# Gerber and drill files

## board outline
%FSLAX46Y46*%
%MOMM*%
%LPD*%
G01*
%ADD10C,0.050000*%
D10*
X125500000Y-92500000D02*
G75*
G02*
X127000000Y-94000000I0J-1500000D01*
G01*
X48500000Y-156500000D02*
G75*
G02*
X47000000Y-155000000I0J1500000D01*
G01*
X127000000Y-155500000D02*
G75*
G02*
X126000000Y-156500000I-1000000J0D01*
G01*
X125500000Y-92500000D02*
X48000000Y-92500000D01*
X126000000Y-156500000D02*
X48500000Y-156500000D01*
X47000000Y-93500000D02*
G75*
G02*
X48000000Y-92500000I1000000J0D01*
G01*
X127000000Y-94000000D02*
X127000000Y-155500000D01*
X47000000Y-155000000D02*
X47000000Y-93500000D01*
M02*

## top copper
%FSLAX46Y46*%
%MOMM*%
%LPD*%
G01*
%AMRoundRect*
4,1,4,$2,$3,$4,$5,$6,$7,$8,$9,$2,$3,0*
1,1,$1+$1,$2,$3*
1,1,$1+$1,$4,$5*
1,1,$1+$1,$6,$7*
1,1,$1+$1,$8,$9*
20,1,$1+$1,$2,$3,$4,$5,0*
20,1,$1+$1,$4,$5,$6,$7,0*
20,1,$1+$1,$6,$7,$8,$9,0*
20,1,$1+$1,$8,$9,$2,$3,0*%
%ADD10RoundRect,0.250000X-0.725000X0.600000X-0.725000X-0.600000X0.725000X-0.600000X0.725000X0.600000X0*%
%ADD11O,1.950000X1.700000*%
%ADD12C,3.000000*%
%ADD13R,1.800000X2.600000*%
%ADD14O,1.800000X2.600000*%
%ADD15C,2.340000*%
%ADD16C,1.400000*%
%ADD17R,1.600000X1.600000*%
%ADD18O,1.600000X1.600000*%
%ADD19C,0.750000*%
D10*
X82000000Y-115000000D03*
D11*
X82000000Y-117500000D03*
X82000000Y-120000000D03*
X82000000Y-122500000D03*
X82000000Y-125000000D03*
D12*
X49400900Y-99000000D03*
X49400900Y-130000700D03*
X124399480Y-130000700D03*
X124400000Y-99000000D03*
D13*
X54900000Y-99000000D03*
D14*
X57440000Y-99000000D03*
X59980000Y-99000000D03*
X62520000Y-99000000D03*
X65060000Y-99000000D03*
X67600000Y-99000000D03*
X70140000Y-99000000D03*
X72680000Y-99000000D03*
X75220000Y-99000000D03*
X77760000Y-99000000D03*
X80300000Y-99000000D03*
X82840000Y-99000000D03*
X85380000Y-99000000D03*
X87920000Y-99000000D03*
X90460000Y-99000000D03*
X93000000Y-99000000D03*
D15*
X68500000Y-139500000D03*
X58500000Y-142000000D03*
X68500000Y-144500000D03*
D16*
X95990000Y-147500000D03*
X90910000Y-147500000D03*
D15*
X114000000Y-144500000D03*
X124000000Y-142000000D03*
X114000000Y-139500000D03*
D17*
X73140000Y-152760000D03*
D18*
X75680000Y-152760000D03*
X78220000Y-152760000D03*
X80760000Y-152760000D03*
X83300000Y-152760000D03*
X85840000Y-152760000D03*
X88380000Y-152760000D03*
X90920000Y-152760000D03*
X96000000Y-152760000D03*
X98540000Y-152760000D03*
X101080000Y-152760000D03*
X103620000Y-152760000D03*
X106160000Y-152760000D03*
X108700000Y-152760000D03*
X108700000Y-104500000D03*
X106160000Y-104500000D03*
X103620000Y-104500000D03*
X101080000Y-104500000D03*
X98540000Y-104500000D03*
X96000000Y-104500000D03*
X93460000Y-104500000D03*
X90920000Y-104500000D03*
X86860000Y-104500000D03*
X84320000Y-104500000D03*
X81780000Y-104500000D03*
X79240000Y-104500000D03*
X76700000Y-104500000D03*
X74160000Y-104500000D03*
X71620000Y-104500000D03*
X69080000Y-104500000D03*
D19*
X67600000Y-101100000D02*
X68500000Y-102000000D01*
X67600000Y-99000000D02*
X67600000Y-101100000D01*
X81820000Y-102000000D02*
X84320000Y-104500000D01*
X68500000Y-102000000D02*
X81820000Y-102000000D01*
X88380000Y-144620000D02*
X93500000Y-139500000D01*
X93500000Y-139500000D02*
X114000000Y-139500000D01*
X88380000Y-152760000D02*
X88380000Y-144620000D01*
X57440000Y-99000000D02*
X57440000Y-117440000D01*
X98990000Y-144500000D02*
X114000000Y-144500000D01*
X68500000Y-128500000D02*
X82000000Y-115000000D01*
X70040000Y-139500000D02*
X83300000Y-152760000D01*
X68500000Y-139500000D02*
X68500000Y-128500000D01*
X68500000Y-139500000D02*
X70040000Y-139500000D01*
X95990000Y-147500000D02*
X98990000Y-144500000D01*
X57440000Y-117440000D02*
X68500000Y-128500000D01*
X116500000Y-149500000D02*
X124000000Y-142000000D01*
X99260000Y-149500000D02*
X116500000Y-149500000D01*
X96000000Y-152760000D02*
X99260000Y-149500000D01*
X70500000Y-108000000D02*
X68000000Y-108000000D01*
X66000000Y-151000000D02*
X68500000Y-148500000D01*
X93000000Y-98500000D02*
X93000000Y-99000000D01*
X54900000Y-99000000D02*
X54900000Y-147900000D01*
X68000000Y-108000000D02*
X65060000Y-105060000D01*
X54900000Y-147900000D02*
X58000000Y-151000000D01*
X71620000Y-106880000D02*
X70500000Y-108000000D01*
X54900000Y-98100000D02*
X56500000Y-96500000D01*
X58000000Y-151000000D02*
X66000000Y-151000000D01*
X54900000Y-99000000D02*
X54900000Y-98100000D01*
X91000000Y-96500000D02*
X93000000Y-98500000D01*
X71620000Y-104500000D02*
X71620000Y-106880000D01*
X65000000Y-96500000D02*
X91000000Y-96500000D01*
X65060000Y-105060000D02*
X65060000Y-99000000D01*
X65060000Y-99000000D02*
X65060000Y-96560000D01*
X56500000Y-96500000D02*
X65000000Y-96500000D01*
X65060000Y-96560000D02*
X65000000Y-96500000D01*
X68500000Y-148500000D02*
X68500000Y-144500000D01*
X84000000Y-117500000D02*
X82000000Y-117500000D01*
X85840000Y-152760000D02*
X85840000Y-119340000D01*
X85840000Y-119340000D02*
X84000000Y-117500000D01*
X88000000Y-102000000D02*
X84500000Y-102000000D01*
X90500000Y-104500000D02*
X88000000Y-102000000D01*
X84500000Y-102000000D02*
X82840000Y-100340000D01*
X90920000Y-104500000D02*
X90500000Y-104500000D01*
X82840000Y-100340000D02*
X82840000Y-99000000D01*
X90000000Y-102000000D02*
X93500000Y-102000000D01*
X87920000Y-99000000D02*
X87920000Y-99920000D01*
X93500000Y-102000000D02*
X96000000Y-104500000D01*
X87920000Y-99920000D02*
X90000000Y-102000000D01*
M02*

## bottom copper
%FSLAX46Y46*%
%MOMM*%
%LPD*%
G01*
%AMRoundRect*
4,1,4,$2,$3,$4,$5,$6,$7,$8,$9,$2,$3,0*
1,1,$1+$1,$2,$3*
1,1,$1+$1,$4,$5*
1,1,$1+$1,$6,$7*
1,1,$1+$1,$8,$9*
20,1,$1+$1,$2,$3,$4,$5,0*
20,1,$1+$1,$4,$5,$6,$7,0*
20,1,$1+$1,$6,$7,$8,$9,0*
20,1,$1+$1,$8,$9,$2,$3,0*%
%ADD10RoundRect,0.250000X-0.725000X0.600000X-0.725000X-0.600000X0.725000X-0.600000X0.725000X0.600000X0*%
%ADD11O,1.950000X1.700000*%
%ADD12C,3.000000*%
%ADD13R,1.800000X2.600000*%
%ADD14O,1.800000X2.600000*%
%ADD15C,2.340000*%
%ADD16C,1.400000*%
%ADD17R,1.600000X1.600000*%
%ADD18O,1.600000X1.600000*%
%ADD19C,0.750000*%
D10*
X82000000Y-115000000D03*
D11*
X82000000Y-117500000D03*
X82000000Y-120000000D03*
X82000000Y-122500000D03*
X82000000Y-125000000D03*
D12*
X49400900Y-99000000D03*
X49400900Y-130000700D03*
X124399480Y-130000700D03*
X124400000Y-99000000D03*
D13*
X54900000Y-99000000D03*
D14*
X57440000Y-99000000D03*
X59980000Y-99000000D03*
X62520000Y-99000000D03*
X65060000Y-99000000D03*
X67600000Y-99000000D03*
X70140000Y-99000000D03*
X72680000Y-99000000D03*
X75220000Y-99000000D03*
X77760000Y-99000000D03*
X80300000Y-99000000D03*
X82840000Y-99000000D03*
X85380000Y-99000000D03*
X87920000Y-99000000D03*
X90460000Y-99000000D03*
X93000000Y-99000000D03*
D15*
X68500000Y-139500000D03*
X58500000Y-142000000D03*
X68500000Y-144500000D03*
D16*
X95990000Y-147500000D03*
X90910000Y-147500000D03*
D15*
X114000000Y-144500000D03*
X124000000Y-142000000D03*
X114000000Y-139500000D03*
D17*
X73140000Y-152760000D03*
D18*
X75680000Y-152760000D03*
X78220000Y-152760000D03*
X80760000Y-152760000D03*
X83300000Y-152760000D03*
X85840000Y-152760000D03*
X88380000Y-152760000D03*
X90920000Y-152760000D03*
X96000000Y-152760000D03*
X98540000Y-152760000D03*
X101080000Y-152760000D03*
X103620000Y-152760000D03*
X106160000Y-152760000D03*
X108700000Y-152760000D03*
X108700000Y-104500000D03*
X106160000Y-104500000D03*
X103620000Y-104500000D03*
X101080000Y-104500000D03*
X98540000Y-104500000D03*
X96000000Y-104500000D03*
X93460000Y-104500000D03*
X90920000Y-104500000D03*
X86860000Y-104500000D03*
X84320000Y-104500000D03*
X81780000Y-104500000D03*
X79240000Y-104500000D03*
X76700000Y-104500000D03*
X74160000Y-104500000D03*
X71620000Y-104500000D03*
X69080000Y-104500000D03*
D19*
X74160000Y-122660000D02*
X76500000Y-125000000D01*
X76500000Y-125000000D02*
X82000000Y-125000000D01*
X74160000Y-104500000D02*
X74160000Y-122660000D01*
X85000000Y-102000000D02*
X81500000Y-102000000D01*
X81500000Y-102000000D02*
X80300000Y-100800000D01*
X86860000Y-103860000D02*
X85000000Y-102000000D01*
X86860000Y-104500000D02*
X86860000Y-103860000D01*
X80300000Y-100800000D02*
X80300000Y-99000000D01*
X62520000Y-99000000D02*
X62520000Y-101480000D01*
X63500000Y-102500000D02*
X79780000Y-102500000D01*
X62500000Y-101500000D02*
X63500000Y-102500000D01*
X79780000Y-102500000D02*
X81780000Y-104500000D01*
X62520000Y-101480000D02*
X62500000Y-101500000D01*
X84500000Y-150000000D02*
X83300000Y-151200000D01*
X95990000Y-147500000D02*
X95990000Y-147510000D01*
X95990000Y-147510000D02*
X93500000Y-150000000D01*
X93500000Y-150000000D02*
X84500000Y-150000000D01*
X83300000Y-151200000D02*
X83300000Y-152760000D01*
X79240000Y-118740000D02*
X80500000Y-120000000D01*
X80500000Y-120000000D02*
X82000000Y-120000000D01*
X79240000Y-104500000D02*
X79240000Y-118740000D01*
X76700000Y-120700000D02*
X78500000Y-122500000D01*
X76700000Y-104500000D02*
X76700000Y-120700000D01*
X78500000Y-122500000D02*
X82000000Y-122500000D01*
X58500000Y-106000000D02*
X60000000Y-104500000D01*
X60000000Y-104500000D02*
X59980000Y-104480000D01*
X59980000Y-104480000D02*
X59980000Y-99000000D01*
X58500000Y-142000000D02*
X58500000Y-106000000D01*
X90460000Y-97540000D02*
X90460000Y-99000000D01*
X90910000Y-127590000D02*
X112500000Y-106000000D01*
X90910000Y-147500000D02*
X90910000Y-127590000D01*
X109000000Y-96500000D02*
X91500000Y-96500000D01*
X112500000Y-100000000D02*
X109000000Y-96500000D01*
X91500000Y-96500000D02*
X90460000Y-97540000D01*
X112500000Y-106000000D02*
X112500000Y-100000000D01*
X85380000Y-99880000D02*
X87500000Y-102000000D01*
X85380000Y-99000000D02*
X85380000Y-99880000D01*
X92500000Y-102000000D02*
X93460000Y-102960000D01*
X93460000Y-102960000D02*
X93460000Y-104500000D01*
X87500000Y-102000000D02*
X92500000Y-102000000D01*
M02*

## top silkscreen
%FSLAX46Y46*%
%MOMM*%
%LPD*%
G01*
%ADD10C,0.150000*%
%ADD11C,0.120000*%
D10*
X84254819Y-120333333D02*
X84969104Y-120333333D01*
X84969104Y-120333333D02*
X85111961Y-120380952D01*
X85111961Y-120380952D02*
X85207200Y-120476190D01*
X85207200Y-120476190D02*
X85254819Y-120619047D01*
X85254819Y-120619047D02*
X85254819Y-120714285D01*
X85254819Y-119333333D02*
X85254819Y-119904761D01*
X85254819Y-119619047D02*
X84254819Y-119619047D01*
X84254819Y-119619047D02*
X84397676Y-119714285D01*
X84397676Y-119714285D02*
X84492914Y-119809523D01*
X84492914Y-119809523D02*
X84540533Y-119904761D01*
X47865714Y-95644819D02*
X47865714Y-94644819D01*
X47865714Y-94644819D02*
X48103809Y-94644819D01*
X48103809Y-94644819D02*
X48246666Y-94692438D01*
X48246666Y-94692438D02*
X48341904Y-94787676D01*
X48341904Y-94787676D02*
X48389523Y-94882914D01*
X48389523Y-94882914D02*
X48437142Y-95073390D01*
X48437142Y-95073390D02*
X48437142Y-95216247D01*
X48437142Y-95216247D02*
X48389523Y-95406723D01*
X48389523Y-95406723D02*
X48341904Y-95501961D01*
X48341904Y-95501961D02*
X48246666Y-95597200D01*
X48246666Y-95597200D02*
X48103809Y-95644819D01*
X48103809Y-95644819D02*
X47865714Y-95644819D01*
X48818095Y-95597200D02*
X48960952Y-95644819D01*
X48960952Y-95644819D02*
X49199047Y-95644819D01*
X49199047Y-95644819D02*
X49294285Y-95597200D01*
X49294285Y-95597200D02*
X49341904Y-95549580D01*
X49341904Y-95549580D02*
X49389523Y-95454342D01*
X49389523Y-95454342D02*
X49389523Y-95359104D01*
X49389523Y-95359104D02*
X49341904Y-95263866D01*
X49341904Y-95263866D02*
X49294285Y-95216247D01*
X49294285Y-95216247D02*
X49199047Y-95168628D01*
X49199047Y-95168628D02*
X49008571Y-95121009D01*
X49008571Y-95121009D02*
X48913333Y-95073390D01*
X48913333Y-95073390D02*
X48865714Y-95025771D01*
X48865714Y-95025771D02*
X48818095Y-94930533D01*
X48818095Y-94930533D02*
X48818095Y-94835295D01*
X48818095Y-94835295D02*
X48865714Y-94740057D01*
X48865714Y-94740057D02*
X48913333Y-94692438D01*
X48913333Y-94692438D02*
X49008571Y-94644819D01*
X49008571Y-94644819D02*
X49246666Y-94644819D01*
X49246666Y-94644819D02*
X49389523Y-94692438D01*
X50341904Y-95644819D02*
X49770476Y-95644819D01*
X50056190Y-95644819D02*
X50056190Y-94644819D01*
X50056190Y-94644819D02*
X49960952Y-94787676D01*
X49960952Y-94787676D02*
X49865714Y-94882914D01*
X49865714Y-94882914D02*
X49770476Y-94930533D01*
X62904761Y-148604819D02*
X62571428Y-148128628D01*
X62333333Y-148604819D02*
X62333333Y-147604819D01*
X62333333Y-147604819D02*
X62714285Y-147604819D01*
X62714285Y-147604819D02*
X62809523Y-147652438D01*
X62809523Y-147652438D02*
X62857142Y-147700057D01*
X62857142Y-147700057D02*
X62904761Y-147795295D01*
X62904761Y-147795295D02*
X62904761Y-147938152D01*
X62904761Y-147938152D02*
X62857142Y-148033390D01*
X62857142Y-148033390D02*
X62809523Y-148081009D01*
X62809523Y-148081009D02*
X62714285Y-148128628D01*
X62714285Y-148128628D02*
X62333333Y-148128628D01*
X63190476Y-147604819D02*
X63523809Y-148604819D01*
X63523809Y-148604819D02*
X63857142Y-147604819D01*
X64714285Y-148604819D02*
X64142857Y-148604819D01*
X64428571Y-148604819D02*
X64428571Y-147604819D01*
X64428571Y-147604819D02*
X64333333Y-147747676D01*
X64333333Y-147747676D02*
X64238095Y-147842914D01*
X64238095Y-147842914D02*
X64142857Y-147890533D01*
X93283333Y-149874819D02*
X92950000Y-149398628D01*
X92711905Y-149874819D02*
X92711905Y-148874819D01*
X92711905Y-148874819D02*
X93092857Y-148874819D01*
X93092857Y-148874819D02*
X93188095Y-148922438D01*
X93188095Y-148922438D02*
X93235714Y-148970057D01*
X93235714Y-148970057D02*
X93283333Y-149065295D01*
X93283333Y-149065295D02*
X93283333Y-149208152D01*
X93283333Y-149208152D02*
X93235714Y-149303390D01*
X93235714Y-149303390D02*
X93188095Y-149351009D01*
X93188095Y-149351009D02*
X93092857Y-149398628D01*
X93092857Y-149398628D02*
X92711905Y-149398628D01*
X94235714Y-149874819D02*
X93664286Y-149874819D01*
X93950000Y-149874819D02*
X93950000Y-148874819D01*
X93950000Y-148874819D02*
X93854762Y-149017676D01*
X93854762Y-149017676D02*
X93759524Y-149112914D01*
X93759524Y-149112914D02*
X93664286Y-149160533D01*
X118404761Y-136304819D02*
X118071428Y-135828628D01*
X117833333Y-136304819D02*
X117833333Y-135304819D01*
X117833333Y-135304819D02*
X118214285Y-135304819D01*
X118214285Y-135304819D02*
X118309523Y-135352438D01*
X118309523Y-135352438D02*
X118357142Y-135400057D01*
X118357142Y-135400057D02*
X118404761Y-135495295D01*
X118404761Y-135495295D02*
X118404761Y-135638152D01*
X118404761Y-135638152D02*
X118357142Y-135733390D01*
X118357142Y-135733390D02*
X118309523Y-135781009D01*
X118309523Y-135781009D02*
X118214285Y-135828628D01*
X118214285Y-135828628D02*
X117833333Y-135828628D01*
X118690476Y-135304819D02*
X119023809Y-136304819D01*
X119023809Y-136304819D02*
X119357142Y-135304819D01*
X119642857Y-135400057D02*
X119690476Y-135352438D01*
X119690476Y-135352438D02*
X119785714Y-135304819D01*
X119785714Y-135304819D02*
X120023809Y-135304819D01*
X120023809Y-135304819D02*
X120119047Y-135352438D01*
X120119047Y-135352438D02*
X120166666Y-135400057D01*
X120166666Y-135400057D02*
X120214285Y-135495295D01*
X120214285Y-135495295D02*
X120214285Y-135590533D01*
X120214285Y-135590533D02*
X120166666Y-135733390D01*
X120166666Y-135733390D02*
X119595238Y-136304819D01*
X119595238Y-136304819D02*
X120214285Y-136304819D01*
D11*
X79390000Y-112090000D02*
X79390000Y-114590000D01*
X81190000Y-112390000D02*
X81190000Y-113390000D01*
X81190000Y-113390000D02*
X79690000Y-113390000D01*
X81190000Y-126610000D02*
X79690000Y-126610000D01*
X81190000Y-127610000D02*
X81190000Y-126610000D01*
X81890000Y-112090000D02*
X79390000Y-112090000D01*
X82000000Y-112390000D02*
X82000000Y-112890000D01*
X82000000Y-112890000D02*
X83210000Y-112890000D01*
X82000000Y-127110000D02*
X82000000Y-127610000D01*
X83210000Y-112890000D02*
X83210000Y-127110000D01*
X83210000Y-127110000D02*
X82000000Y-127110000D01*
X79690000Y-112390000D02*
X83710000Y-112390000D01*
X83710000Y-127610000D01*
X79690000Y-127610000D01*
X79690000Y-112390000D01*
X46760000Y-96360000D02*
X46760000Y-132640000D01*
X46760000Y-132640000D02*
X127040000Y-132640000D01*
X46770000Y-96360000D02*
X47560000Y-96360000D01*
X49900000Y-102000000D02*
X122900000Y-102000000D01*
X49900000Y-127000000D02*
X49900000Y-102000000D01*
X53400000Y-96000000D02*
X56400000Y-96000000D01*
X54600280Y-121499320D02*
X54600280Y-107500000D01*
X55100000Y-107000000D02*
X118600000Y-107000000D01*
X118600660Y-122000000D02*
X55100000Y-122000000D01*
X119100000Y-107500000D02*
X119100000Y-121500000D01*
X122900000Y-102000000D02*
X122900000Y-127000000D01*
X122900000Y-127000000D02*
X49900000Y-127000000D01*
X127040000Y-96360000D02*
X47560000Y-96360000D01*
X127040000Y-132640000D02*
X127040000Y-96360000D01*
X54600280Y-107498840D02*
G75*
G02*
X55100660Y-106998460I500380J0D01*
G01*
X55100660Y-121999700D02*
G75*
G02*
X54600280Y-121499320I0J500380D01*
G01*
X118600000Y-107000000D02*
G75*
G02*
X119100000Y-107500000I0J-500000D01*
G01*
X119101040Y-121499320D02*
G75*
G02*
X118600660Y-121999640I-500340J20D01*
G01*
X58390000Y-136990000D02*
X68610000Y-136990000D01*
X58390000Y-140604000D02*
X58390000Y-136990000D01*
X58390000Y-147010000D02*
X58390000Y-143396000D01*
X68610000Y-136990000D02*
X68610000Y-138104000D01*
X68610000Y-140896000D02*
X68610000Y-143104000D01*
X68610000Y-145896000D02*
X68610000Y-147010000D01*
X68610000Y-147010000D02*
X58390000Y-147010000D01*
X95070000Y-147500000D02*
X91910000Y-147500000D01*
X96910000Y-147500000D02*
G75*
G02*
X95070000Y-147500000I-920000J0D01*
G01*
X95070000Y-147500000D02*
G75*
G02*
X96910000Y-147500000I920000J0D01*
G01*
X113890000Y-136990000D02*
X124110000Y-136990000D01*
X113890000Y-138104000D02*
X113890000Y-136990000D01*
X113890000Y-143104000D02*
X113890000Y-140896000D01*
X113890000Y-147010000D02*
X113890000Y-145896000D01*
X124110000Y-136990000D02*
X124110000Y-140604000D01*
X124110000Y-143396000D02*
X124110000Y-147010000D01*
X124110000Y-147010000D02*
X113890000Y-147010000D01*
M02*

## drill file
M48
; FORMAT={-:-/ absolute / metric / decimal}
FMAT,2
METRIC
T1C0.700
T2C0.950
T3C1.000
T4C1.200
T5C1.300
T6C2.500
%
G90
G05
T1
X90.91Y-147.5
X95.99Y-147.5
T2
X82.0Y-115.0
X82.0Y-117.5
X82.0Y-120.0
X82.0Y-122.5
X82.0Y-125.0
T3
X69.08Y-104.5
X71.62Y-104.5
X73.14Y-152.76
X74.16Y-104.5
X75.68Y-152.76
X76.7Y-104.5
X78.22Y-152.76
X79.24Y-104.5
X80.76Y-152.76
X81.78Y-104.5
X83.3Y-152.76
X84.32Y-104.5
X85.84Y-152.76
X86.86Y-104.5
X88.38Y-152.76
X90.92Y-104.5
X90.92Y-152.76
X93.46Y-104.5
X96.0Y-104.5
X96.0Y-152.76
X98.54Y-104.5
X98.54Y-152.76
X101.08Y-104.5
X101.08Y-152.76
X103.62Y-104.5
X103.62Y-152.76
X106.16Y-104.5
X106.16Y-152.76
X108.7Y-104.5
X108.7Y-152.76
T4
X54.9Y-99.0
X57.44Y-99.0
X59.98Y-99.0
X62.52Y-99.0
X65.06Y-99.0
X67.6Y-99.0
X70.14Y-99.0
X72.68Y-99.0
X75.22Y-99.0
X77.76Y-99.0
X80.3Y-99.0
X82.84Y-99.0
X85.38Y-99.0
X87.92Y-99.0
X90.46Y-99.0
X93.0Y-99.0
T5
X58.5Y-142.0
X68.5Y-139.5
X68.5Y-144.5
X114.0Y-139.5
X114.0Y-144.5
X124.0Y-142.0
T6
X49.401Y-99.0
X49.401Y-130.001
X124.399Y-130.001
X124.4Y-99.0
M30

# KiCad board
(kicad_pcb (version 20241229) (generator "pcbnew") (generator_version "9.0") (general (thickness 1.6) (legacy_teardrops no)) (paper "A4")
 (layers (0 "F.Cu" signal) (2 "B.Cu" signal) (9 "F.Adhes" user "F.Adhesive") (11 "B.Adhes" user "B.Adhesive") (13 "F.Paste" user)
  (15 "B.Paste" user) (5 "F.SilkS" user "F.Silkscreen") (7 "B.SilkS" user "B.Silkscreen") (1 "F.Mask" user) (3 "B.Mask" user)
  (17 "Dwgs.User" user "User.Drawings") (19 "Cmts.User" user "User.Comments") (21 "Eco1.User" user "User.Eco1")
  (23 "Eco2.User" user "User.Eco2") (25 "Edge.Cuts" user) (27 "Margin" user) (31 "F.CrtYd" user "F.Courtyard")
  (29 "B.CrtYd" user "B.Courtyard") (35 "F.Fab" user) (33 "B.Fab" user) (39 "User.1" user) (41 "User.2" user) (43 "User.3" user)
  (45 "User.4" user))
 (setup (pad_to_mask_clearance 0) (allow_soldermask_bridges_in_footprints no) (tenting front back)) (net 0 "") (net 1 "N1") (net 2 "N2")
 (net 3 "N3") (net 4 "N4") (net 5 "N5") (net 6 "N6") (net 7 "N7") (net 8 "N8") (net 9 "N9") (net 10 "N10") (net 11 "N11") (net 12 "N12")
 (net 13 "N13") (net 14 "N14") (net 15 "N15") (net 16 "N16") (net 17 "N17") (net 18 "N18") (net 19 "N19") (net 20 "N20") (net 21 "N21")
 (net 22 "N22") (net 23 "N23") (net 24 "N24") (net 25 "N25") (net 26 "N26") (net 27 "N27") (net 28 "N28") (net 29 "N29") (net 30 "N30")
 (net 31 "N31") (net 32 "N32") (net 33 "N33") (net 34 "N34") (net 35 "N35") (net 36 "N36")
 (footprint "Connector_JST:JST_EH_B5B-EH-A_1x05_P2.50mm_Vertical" (layer "F.Cu") (at 82 115 -90)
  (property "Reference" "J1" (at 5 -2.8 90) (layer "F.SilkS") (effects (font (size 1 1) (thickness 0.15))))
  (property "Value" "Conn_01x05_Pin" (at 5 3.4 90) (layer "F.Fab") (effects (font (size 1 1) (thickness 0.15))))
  (fp_line (start -2.91 2.61) (end -0.41 2.61) (stroke (width 0.12) (type solid)) (layer "F.SilkS"))
  (fp_line (start -2.61 0.81) (end -1.61 0.81) (stroke (width 0.12) (type solid)) (layer "F.SilkS"))
  (fp_line (start -1.61 0.81) (end -1.61 2.31) (stroke (width 0.12) (type solid)) (layer "F.SilkS"))
  (fp_line (start 11.61 0.81) (end 11.61 2.31) (stroke (width 0.12) (type solid)) (layer "F.SilkS"))
  (fp_line (start 12.61 0.81) (end 11.61 0.81) (stroke (width 0.12) (type solid)) (layer "F.SilkS"))
  (fp_line (start -2.91 0.11) (end -2.91 2.61) (stroke (width 0.12) (type solid)) (layer "F.SilkS"))
  (fp_line (start -2.61 0) (end -2.11 0) (stroke (width 0.12) (type solid)) (layer "F.SilkS"))
  (fp_line (start -2.11 0) (end -2.11 -1.21) (stroke (width 0.12) (type solid)) (layer "F.SilkS"))
  (fp_line (start 12.11 0) (end 12.61 0) (stroke (width 0.12) (type solid)) (layer "F.SilkS"))
  (fp_line (start -2.11 -1.21) (end 12.11 -1.21) (stroke (width 0.12) (type solid)) (layer "F.SilkS"))
  (fp_line (start 12.11 -1.21) (end 12.11 0) (stroke (width 0.12) (type solid)) (layer "F.SilkS"))
  (fp_rect (start -2.61 -1.71) (end 12.61 2.31) (stroke (width 0.12) (type solid)) (fill no) (layer "F.SilkS"))
  (pad "1" thru_hole roundrect (at 0 0 270) (size 1.7 1.95) (drill 0.95) (layers "*.Cu" "*.Mask") (remove_unused_layers no)
   (roundrect_rratio 0.147059) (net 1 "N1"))
  (pad "2" thru_hole oval (at 2.5 0 270) (size 1.7 1.95) (drill 0.95) (layers "*.Cu" "*.Mask") (remove_unused_layers no) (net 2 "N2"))
  (pad "3" thru_hole oval (at 5 0 270) (size 1.7 1.95) (drill 0.95) (layers "*.Cu" "*.Mask") (remove_unused_layers no) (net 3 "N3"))
  (pad "4" thru_hole oval (at 7.5 0 270) (size 1.7 1.95) (drill 0.95) (layers "*.Cu" "*.Mask") (remove_unused_layers no) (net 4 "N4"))
  (pad "5" thru_hole oval (at 10 0 270) (size 1.7 1.95) (drill 0.95) (layers "*.Cu" "*.Mask") (remove_unused_layers no) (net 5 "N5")))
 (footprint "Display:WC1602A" (layer "F.Cu") (at 54.9 99)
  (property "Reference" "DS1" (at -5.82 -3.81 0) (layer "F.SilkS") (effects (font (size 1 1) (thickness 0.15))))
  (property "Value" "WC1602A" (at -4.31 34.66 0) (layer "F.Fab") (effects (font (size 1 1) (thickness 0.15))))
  (fp_line (start -8.14 -2.64) (end -8.14 33.64) (stroke (width 0.12) (type solid)) (layer "F.SilkS"))
  (fp_line (start -8.14 33.64) (end 72.14 33.64) (stroke (width 0.12) (type solid)) (layer "F.SilkS"))
  (fp_line (start -8.13 -2.64) (end -7.34 -2.64) (stroke (width 0.12) (type solid)) (layer "F.SilkS"))
  (fp_line (start -5 3) (end 68 3) (stroke (width 0.12) (type solid)) (layer "F.SilkS"))
  (fp_line (start -5 28) (end -5 3) (stroke (width 0.12) (type solid)) (layer "F.SilkS"))
  (fp_line (start -1.5 -3) (end 1.5 -3) (stroke (width 0.12) (type solid)) (layer "F.SilkS"))
  (fp_line (start -0.29972 22.49932) (end -0.29972 8.5) (stroke (width 0.12) (type solid)) (layer "F.SilkS"))
  (fp_line (start 0.2 8) (end 63.7 8) (stroke (width 0.12) (type solid)) (layer "F.SilkS"))
  (fp_line (start 63.70066 23) (end 0.2 23) (stroke (width 0.12) (type solid)) (layer "F.SilkS"))
  (fp_line (start 64.2 8.5) (end 64.2 22.5) (stroke (width 0.12) (type solid)) (layer "F.SilkS"))
  (fp_line (start 68 3) (end 68 28) (stroke (width 0.12) (type solid)) (layer "F.SilkS"))
  (fp_line (start 68 28) (end -5 28) (stroke (width 0.12) (type solid)) (layer "F.SilkS"))
  (fp_line (start 72.14 -2.64) (end -7.34 -2.64) (stroke (width 0.12) (type solid)) (layer "F.SilkS"))
  (fp_line (start 72.14 33.64) (end 72.14 -2.64) (stroke (width 0.12) (type solid)) (layer "F.SilkS"))
  (fp_arc (start -0.29972 8.49884) (mid -0.153162 8.145018) (end 0.20066 7.99846) (stroke (width 0.12) (type solid)) (layer "F.SilkS"))
  (fp_arc (start 0.20066 22.9997) (mid -0.153162 22.853142) (end -0.29972 22.49932) (stroke (width 0.12) (type solid)) (layer "F.SilkS"))
  (fp_arc (start 63.7 8) (mid 64.053553 8.146447) (end 64.2 8.5) (stroke (width 0.12) (type solid)) (layer "F.SilkS"))
  (fp_arc (start 64.20104 22.49932) (mid 64.054482 22.853142) (end 63.70066 22.9997) (stroke (width 0.12) (type solid)) (layer "F.SilkS"))
  (pad "" thru_hole circle (at -5.4991 0) (size 3 3) (drill 2.5) (layers "*.Cu" "*.Mask") (remove_unused_layers no))
  (pad "" thru_hole circle (at -5.4991 31.0007) (size 3 3) (drill 2.5) (layers "*.Cu" "*.Mask") (remove_unused_layers no))
  (pad "" thru_hole circle (at 69.49948 31.0007) (size 3 3) (drill 2.5) (layers "*.Cu" "*.Mask") (remove_unused_layers no))
  (pad "" thru_hole circle (at 69.5 0) (size 3 3) (drill 2.5) (layers "*.Cu" "*.Mask") (remove_unused_layers no))
  (pad "1" thru_hole rect (at 0 0) (size 1.8 2.6) (drill 1.2) (layers "*.Cu" "*.Mask") (remove_unused_layers no) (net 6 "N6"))
  (pad "2" thru_hole oval (at 2.54 0) (size 1.8 2.6) (drill 1.2) (layers "*.Cu" "*.Mask") (remove_unused_layers no) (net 1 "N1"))
  (pad "3" thru_hole oval (at 5.08 0) (size 1.8 2.6) (drill 1.2) (layers "*.Cu" "*.Mask") (remove_unused_layers no) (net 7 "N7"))
  (pad "4" thru_hole oval (at 7.62 0) (size 1.8 2.6) (drill 1.2) (layers "*.Cu" "*.Mask") (remove_unused_layers no) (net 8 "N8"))
  (pad "5" thru_hole oval (at 10.16 0) (size 1.8 2.6) (drill 1.2) (layers "*.Cu" "*.Mask") (remove_unused_layers no) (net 6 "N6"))
  (pad "6" thru_hole oval (at 12.7 0) (size 1.8 2.6) (drill 1.2) (layers "*.Cu" "*.Mask") (remove_unused_layers no) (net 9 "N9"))
  (pad "7" thru_hole oval (at 15.24 0) (size 1.8 2.6) (drill 1.2) (layers "*.Cu" "*.Mask") (remove_unused_layers no) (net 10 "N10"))
  (pad "8" thru_hole oval (at 17.78 0) (size 1.8 2.6) (drill 1.2) (layers "*.Cu" "*.Mask") (remove_unused_layers no) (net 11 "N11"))
  (pad "9" thru_hole oval (at 20.32 0) (size 1.8 2.6) (drill 1.2) (layers "*.Cu" "*.Mask") (remove_unused_layers no) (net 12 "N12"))
  (pad "10" thru_hole oval (at 22.86 0) (size 1.8 2.6) (drill 1.2) (layers "*.Cu" "*.Mask") (remove_unused_layers no) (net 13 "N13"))
  (pad "11" thru_hole oval (at 25.4 0) (size 1.8 2.6) (drill 1.2) (layers "*.Cu" "*.Mask") (remove_unused_layers no) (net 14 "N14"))
  (pad "12" thru_hole oval (at 27.94 0) (size 1.8 2.6) (drill 1.2) (layers "*.Cu" "*.Mask") (remove_unused_layers no) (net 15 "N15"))
  (pad "13" thru_hole oval (at 30.48 0) (size 1.8 2.6) (drill 1.2) (layers "*.Cu" "*.Mask") (remove_unused_layers no) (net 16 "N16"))
  (pad "14" thru_hole oval (at 33.02 0) (size 1.8 2.6) (drill 1.2) (layers "*.Cu" "*.Mask") (remove_unused_layers no) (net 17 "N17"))
  (pad "15" thru_hole oval (at 35.56 0) (size 1.8 2.6) (drill 1.2) (layers "*.Cu" "*.Mask") (remove_unused_layers no) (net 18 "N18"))
  (pad "16" thru_hole oval (at 38.1 0) (size 1.8 2.6) (drill 1.2) (layers "*.Cu" "*.Mask") (remove_unused_layers no) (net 6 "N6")))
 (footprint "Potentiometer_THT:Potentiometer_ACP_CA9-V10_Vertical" (layer "F.Cu") (at 68.5 139.5 180)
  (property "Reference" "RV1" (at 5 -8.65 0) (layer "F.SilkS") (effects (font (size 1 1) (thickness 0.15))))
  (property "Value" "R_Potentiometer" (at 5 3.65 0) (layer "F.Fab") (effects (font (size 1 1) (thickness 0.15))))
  (fp_line (start 10.11 2.51) (end -0.11 2.51) (stroke (width 0.12) (type solid)) (layer "F.SilkS"))
  (fp_line (start 10.11 -1.104) (end 10.11 2.51) (stroke (width 0.12) (type solid)) (layer "F.SilkS"))
  (fp_line (start 10.11 -7.51) (end 10.11 -3.896) (stroke (width 0.12) (type solid)) (layer "F.SilkS"))
  (fp_line (start -0.11 2.51) (end -0.11 1.396) (stroke (width 0.12) (type solid)) (layer "F.SilkS"))
  (fp_line (start -0.11 -1.396) (end -0.11 -3.604) (stroke (width 0.12) (type solid)) (layer "F.SilkS"))
  (fp_line (start -0.11 -6.396) (end -0.11 -7.51) (stroke (width 0.12) (type solid)) (layer "F.SilkS"))
  (fp_line (start -0.11 -7.51) (end 10.11 -7.51) (stroke (width 0.12) (type solid)) (layer "F.SilkS"))
  (pad "1" thru_hole circle (at 0 0 180) (size 2.34 2.34) (drill 1.3) (layers "*.Cu" "*.Mask") (remove_unused_layers no) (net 1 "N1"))
  (pad "2" thru_hole circle (at 10 -2.5 180) (size 2.34 2.34) (drill 1.3) (layers "*.Cu" "*.Mask") (remove_unused_layers no) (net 7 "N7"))
  (pad "3" thru_hole circle (at 0 -5 180) (size 2.34 2.34) (drill 1.3) (layers "*.Cu" "*.Mask") (remove_unused_layers no) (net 6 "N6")))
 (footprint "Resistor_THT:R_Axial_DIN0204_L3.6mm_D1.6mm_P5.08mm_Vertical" (layer "F.Cu") (at 95.99 147.5 180)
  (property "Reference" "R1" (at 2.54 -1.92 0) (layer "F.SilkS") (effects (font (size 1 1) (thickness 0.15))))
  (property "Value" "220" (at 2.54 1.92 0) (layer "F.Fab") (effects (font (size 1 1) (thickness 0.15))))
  (fp_line (start 0.92 0) (end 4.08 0) (stroke (width 0.12) (type solid)) (layer "F.SilkS"))
  (fp_circle (center 0 0) (end 0.92 0) (stroke (width 0.12) (type solid)) (fill no) (layer "F.SilkS"))
  (pad "1" thru_hole circle (at 0 0 180) (size 1.4 1.4) (drill 0.7) (layers "*.Cu" "*.Mask") (remove_unused_layers no) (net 1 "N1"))
  (pad "2" thru_hole circle (at 5.08 0 180) (size 1.4 1.4) (drill 0.7) (layers "*.Cu" "*.Mask") (remove_unused_layers no) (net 18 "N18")))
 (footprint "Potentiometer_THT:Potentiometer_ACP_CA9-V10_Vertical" (layer "F.Cu") (at 114 144.5)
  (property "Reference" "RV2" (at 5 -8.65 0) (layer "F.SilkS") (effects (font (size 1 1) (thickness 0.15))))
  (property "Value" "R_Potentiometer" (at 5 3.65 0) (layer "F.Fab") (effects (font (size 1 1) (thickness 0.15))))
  (fp_line (start -0.11 -7.51) (end 10.11 -7.51) (stroke (width 0.12) (type solid)) (layer "F.SilkS"))
  (fp_line (start -0.11 -6.396) (end -0.11 -7.51) (stroke (width 0.12) (type solid)) (layer "F.SilkS"))
  (fp_line (start -0.11 -1.396) (end -0.11 -3.604) (stroke (width 0.12) (type solid)) (layer "F.SilkS"))
  (fp_line (start -0.11 2.51) (end -0.11 1.396) (stroke (width 0.12) (type solid)) (layer "F.SilkS"))
  (fp_line (start 10.11 -7.51) (end 10.11 -3.896) (stroke (width 0.12) (type solid)) (layer "F.SilkS"))
  (fp_line (start 10.11 -1.104) (end 10.11 2.51) (stroke (width 0.12) (type solid)) (layer "F.SilkS"))
  (fp_line (start 10.11 2.51) (end -0.11 2.51) (stroke (width 0.12) (type solid)) (layer "F.SilkS"))
  (pad "1" thru_hole circle (at 0 0) (size 2.34 2.34) (drill 1.3) (layers "*.Cu" "*.Mask") (remove_unused_layers no) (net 1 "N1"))
  (pad "2" thru_hole circle (at 10 -2.5) (size 2.34 2.34) (drill 1.3) (layers "*.Cu" "*.Mask") (remove_unused_layers no) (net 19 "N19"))
  (pad "3" thru_hole circle (at 0 -5) (size 2.34 2.34) (drill 1.3) (layers "*.Cu" "*.Mask") (remove_unused_layers no) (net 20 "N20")))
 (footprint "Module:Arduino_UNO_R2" (layer "B.Cu") (at 73.14 152.76)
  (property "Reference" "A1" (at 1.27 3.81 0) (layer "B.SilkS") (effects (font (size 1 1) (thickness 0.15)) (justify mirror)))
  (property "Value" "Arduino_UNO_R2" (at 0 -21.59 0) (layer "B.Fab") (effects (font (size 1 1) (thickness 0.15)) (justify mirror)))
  (pad "1" thru_hole rect (at 0 0 270) (size 1.6 1.6) (drill 1) (layers "*.Cu" "*.Mask") (remove_unused_layers no) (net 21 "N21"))
  (pad "2" thru_hole oval (at 2.54 0 270) (size 1.6 1.6) (drill 1) (layers "*.Cu" "*.Mask") (remove_unused_layers no) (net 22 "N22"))
  (pad "3" thru_hole oval (at 5.08 0 270) (size 1.6 1.6) (drill 1) (layers "*.Cu" "*.Mask") (remove_unused_layers no) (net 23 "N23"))
  (pad "4" thru_hole oval (at 7.62 0 270) (size 1.6 1.6) (drill 1) (layers "*.Cu" "*.Mask") (remove_unused_layers no) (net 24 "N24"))
  (pad "5" thru_hole oval (at 10.16 0 270) (size 1.6 1.6) (drill 1) (layers "*.Cu" "*.Mask") (remove_unused_layers no) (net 1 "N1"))
  (pad "6" thru_hole oval (at 12.7 0 270) (size 1.6 1.6) (drill 1) (layers "*.Cu" "*.Mask") (remove_unused_layers no) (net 2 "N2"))
  (pad "7" thru_hole oval (at 15.24 0 270) (size 1.6 1.6) (drill 1) (layers "*.Cu" "*.Mask") (remove_unused_layers no) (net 20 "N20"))
  (pad "8" thru_hole oval (at 17.78 0 270) (size 1.6 1.6) (drill 1) (layers "*.Cu" "*.Mask") (remove_unused_layers no) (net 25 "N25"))
  (pad "9" thru_hole oval (at 22.86 0 270) (size 1.6 1.6) (drill 1) (layers "*.Cu" "*.Mask") (remove_unused_layers no) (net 19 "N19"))
  (pad "10" thru_hole oval (at 25.4 0 270) (size 1.6 1.6) (drill 1) (layers "*.Cu" "*.Mask") (remove_unused_layers no) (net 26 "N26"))
  (pad "11" thru_hole oval (at 27.94 0 270) (size 1.6 1.6) (drill 1) (layers "*.Cu" "*.Mask") (remove_unused_layers no) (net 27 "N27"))
  (pad "12" thru_hole oval (at 30.48 0 270) (size 1.6 1.6) (drill 1) (layers "*.Cu" "*.Mask") (remove_unused_layers no) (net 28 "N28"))
  (pad "13" thru_hole oval (at 33.02 0 270) (size 1.6 1.6) (drill 1) (layers "*.Cu" "*.Mask") (remove_unused_layers no) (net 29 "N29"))
  (pad "14" thru_hole oval (at 35.56 0 270) (size 1.6 1.6) (drill 1) (layers "*.Cu" "*.Mask") (remove_unused_layers no) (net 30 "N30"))
  (pad "15" thru_hole oval (at 35.56 -48.26 270) (size 1.6 1.6) (drill 1) (layers "*.Cu" "*.Mask") (remove_unused_layers no) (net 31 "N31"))
  (pad "16" thru_hole oval (at 33.02 -48.26 270) (size 1.6 1.6) (drill 1) (layers "*.Cu" "*.Mask") (remove_unused_layers no) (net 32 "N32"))
  (pad "17" thru_hole oval (at 30.48 -48.26 270) (size 1.6 1.6) (drill 1) (layers "*.Cu" "*.Mask") (remove_unused_layers no) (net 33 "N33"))
  (pad "18" thru_hole oval (at 27.94 -48.26 270) (size 1.6 1.6) (drill 1) (layers "*.Cu" "*.Mask") (remove_unused_layers no) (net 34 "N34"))
  (pad "19" thru_hole oval (at 25.4 -48.26 270) (size 1.6 1.6) (drill 1) (layers "*.Cu" "*.Mask") (remove_unused_layers no) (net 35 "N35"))
  (pad "20" thru_hole oval (at 22.86 -48.26 270) (size 1.6 1.6) (drill 1) (layers "*.Cu" "*.Mask") (remove_unused_layers no) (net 17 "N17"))
  (pad "21" thru_hole oval (at 20.32 -48.26 270) (size 1.6 1.6) (drill 1) (layers "*.Cu" "*.Mask") (remove_unused_layers no) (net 16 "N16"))
  (pad "22" thru_hole oval (at 17.78 -48.26 270) (size 1.6 1.6) (drill 1) (layers "*.Cu" "*.Mask") (remove_unused_layers no) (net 15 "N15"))
  (pad "23" thru_hole oval (at 13.72 -48.26 270) (size 1.6 1.6) (drill 1) (layers "*.Cu" "*.Mask") (remove_unused_layers no) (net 14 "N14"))
  (pad "24" thru_hole oval (at 11.18 -48.26 270) (size 1.6 1.6) (drill 1) (layers "*.Cu" "*.Mask") (remove_unused_layers no) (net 9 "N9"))
  (pad "25" thru_hole oval (at 8.64 -48.26 270) (size 1.6 1.6) (drill 1) (layers "*.Cu" "*.Mask") (remove_unused_layers no) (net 8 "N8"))
  (pad "26" thru_hole oval (at 6.1 -48.26 270) (size 1.6 1.6) (drill 1) (layers "*.Cu" "*.Mask") (remove_unused_layers no) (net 3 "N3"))
  (pad "27" thru_hole oval (at 3.56 -48.26 270) (size 1.6 1.6) (drill 1) (layers "*.Cu" "*.Mask") (remove_unused_layers no) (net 4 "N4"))
  (pad "28" thru_hole oval (at 1.02 -48.26 270) (size 1.6 1.6) (drill 1) (layers "*.Cu" "*.Mask") (remove_unused_layers no) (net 5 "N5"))
  (pad "29" thru_hole oval (at -1.52 -48.26 270) (size 1.6 1.6) (drill 1) (layers "*.Cu" "*.Mask") (remove_unused_layers no) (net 6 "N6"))
  (pad "30" thru_hole oval (at -4.06 -48.26 270) (size 1.6 1.6) (drill 1) (layers "*.Cu" "*.Mask") (remove_unused_layers no) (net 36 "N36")))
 (gr_arc (start 125.5 92.5) (mid 126.56066 92.93934) (end 127 94) (stroke (width 0.05) (type default)) (layer "Edge.Cuts"))
 (gr_arc (start 48.5 156.5) (mid 47.43934 156.06066) (end 47 155) (stroke (width 0.05) (type default)) (layer "Edge.Cuts"))
 (gr_arc (start 127 155.5) (mid 126.707107 156.207107) (end 126 156.5) (stroke (width 0.05) (type default)) (layer "Edge.Cuts"))
 (gr_line (start 125.5 92.5) (end 48 92.5) (stroke (width 0.05) (type default)) (layer "Edge.Cuts"))
 (gr_line (start 126 156.5) (end 48.5 156.5) (stroke (width 0.05) (type default)) (layer "Edge.Cuts"))
 (gr_arc (start 47 93.5) (mid 47.292893 92.792893) (end 48 92.5) (stroke (width 0.05) (type default)) (layer "Edge.Cuts"))
 (gr_line (start 127 94) (end 127 155.5) (stroke (width 0.05) (type default)) (layer "Edge.Cuts"))
 (gr_line (start 47 155) (end 47 93.5) (stroke (width 0.05) (type default)) (layer "Edge.Cuts"))
 (segment (start 74.16 122.66) (end 76.5 125) (width 0.75) (layer "B.Cu") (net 5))
 (segment (start 76.5 125) (end 82 125) (width 0.75) (layer "B.Cu") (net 5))
 (segment (start 74.16 104.5) (end 74.16 122.66) (width 0.75) (layer "B.Cu") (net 5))
 (segment (start 67.6 101.1) (end 68.5 102) (width 0.75) (layer "F.Cu") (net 9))
 (segment (start 67.6 99) (end 67.6 101.1) (width 0.75) (layer "F.Cu") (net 9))
 (segment (start 81.82 102) (end 84.32 104.5) (width 0.75) (layer "F.Cu") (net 9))
 (segment (start 68.5 102) (end 81.82 102) (width 0.75) (layer "F.Cu") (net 9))
 (segment (start 88.38 144.62) (end 93.5 139.5) (width 0.75) (layer "F.Cu") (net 20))
 (segment (start 93.5 139.5) (end 114 139.5) (width 0.75) (layer "F.Cu") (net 20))
 (segment (start 88.38 152.76) (end 88.38 144.62) (width 0.75) (layer "F.Cu") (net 20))
 (segment (start 85 102) (end 81.5 102) (width 0.75) (layer "B.Cu") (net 14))
 (segment (start 81.5 102) (end 80.3 100.8) (width 0.75) (layer "B.Cu") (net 14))
 (segment (start 86.86 103.86) (end 85 102) (width 0.75) (layer "B.Cu") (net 14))
 (segment (start 86.86 104.5) (end 86.86 103.86) (width 0.75) (layer "B.Cu") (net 14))
 (segment (start 80.3 100.8) (end 80.3 99) (width 0.75) (layer "B.Cu") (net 14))
 (segment (start 62.52 99) (end 62.52 101.48) (width 0.75) (layer "B.Cu") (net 8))
 (segment (start 63.5 102.5) (end 79.78 102.5) (width 0.75) (layer "B.Cu") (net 8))
 (segment (start 62.5 101.5) (end 63.5 102.5) (width 0.75) (layer "B.Cu") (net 8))
 (segment (start 79.78 102.5) (end 81.78 104.5) (width 0.75) (layer "B.Cu") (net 8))
 (segment (start 62.52 101.48) (end 62.5 101.5) (width 0.75) (layer "B.Cu") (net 8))
 (segment (start 57.44 99) (end 57.44 117.44) (width 0.75) (layer "F.Cu") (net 1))
 (segment (start 98.99 144.5) (end 114 144.5) (width 0.75) (layer "F.Cu") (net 1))
 (segment (start 68.5 128.5) (end 82 115) (width 0.75) (layer "F.Cu") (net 1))
 (segment (start 70.04 139.5) (end 83.3 152.76) (width 0.75) (layer "F.Cu") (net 1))
 (segment (start 68.5 139.5) (end 68.5 128.5) (width 0.75) (layer "F.Cu") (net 1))
 (segment (start 68.5 139.5) (end 70.04 139.5) (width 0.75) (layer "F.Cu") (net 1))
 (segment (start 95.99 147.5) (end 98.99 144.5) (width 0.75) (layer "F.Cu") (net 1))
 (segment (start 57.44 117.44) (end 68.5 128.5) (width 0.75) (layer "F.Cu") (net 1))
 (segment (start 84.5 150) (end 83.3 151.2) (width 0.75) (layer "B.Cu") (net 1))
 (segment (start 95.99 147.5) (end 95.99 147.51) (width 0.75) (layer "B.Cu") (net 1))
 (segment (start 95.99 147.51) (end 93.5 150) (width 0.75) (layer "B.Cu") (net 1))
 (segment (start 93.5 150) (end 84.5 150) (width 0.75) (layer "B.Cu") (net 1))
 (segment (start 83.3 151.2) (end 83.3 152.76) (width 0.75) (layer "B.Cu") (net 1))
 (segment (start 116.5 149.5) (end 124 142) (width 0.75) (layer "F.Cu") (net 19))
 (segment (start 99.26 149.5) (end 116.5 149.5) (width 0.75) (layer "F.Cu") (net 19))
 (segment (start 96 152.76) (end 99.26 149.5) (width 0.75) (layer "F.Cu") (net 19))
 (segment (start 79.24 118.74) (end 80.5 120) (width 0.75) (layer "B.Cu") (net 3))
 (segment (start 80.5 120) (end 82 120) (width 0.75) (layer "B.Cu") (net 3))
 (segment (start 79.24 104.5) (end 79.24 118.74) (width 0.75) (layer "B.Cu") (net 3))
 (segment (start 70.5 108) (end 68 108) (width 0.75) (layer "F.Cu") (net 6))
 (segment (start 66 151) (end 68.5 148.5) (width 0.75) (layer "F.Cu") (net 6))
 (segment (start 93 98.5) (end 93 99) (width 0.75) (layer "F.Cu") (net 6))
 (segment (start 54.9 99) (end 54.9 147.9) (width 0.75) (layer "F.Cu") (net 6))
 (segment (start 68 108) (end 65.06 105.06) (width 0.75) (layer "F.Cu") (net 6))
 (segment (start 54.9 147.9) (end 58 151) (width 0.75) (layer "F.Cu") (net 6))
 (segment (start 71.62 106.88) (end 70.5 108) (width 0.75) (layer "F.Cu") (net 6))
 (segment (start 54.9 98.1) (end 56.5 96.5) (width 0.75) (layer "F.Cu") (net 6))
 (segment (start 58 151) (end 66 151) (width 0.75) (layer "F.Cu") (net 6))
 (segment (start 54.9 99) (end 54.9 98.1) (width 0.75) (layer "F.Cu") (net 6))
 (segment (start 91 96.5) (end 93 98.5) (width 0.75) (layer "F.Cu") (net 6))
 (segment (start 71.62 104.5) (end 71.62 106.88) (width 0.75) (layer "F.Cu") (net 6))
 (segment (start 65 96.5) (end 91 96.5) (width 0.75) (layer "F.Cu") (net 6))
 (segment (start 65.06 105.06) (end 65.06 99) (width 0.75) (layer "F.Cu") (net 6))
 (segment (start 65.06 99) (end 65.06 96.56) (width 0.75) (layer "F.Cu") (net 6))
 (segment (start 56.5 96.5) (end 65 96.5) (width 0.75) (layer "F.Cu") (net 6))
 (segment (start 65.06 96.56) (end 65 96.5) (width 0.75) (layer "F.Cu") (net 6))
 (segment (start 68.5 148.5) (end 68.5 144.5) (width 0.75) (layer "F.Cu") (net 6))
 (segment (start 84 117.5) (end 82 117.5) (width 0.75) (layer "F.Cu") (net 2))
 (segment (start 85.84 152.76) (end 85.84 119.34) (width 0.75) (layer "F.Cu") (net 2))
 (segment (start 85.84 119.34) (end 84 117.5) (width 0.75) (layer "F.Cu") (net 2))
 (segment (start 76.7 120.7) (end 78.5 122.5) (width 0.75) (layer "B.Cu") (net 4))
 (segment (start 76.7 104.5) (end 76.7 120.7) (width 0.75) (layer "B.Cu") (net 4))
 (segment (start 78.5 122.5) (end 82 122.5) (width 0.75) (layer "B.Cu") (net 4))
 (segment (start 58.5 106) (end 60 104.5) (width 0.75) (layer "B.Cu") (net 7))
 (segment (start 60 104.5) (end 59.98 104.48) (width 0.75) (layer "B.Cu") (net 7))
 (segment (start 59.98 104.48) (end 59.98 99) (width 0.75) (layer "B.Cu") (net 7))
 (segment (start 58.5 142) (end 58.5 106) (width 0.75) (layer "B.Cu") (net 7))
 (segment (start 90.46 97.54) (end 90.46 99) (width 0.75) (layer "B.Cu") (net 18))
 (segment (start 90.91 127.59) (end 112.5 106) (width 0.75) (layer "B.Cu") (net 18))
 (segment (start 90.91 147.5) (end 90.91 127.59) (width 0.75) (layer "B.Cu") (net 18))
 (segment (start 109 96.5) (end 91.5 96.5) (width 0.75) (layer "B.Cu") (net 18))
 (segment (start 112.5 100) (end 109 96.5) (width 0.75) (layer "B.Cu") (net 18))
 (segment (start 91.5 96.5) (end 90.46 97.54) (width 0.75) (layer "B.Cu") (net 18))
 (segment (start 112.5 106) (end 112.5 100) (width 0.75) (layer "B.Cu") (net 18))
 (segment (start 88 102) (end 84.5 102) (width 0.75) (layer "F.Cu") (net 15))
 (segment (start 90.5 104.5) (end 88 102) (width 0.75) (layer "F.Cu") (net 15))
 (segment (start 84.5 102) (end 82.84 100.34) (width 0.75) (layer "F.Cu") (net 15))
 (segment (start 90.92 104.5) (end 90.5 104.5) (width 0.75) (layer "F.Cu") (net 15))
 (segment (start 82.84 100.34) (end 82.84 99) (width 0.75) (layer "F.Cu") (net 15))
 (segment (start 85.38 99.88) (end 87.5 102) (width 0.75) (layer "B.Cu") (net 16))
 (segment (start 85.38 99) (end 85.38 99.88) (width 0.75) (layer "B.Cu") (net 16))
 (segment (start 92.5 102) (end 93.46 102.96) (width 0.75) (layer "B.Cu") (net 16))
 (segment (start 93.46 102.96) (end 93.46 104.5) (width 0.75) (layer "B.Cu") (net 16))
 (segment (start 87.5 102) (end 92.5 102) (width 0.75) (layer "B.Cu") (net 16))
 (segment (start 90 102) (end 93.5 102) (width 0.75) (layer "F.Cu") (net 17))
 (segment (start 87.92 99) (end 87.92 99.92) (width 0.75) (layer "F.Cu") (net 17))
 (segment (start 93.5 102) (end 96 104.5) (width 0.75) (layer "F.Cu") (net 17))
 (segment (start 87.92 99.92) (end 90 102) (width 0.75) (layer "F.Cu") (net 17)))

